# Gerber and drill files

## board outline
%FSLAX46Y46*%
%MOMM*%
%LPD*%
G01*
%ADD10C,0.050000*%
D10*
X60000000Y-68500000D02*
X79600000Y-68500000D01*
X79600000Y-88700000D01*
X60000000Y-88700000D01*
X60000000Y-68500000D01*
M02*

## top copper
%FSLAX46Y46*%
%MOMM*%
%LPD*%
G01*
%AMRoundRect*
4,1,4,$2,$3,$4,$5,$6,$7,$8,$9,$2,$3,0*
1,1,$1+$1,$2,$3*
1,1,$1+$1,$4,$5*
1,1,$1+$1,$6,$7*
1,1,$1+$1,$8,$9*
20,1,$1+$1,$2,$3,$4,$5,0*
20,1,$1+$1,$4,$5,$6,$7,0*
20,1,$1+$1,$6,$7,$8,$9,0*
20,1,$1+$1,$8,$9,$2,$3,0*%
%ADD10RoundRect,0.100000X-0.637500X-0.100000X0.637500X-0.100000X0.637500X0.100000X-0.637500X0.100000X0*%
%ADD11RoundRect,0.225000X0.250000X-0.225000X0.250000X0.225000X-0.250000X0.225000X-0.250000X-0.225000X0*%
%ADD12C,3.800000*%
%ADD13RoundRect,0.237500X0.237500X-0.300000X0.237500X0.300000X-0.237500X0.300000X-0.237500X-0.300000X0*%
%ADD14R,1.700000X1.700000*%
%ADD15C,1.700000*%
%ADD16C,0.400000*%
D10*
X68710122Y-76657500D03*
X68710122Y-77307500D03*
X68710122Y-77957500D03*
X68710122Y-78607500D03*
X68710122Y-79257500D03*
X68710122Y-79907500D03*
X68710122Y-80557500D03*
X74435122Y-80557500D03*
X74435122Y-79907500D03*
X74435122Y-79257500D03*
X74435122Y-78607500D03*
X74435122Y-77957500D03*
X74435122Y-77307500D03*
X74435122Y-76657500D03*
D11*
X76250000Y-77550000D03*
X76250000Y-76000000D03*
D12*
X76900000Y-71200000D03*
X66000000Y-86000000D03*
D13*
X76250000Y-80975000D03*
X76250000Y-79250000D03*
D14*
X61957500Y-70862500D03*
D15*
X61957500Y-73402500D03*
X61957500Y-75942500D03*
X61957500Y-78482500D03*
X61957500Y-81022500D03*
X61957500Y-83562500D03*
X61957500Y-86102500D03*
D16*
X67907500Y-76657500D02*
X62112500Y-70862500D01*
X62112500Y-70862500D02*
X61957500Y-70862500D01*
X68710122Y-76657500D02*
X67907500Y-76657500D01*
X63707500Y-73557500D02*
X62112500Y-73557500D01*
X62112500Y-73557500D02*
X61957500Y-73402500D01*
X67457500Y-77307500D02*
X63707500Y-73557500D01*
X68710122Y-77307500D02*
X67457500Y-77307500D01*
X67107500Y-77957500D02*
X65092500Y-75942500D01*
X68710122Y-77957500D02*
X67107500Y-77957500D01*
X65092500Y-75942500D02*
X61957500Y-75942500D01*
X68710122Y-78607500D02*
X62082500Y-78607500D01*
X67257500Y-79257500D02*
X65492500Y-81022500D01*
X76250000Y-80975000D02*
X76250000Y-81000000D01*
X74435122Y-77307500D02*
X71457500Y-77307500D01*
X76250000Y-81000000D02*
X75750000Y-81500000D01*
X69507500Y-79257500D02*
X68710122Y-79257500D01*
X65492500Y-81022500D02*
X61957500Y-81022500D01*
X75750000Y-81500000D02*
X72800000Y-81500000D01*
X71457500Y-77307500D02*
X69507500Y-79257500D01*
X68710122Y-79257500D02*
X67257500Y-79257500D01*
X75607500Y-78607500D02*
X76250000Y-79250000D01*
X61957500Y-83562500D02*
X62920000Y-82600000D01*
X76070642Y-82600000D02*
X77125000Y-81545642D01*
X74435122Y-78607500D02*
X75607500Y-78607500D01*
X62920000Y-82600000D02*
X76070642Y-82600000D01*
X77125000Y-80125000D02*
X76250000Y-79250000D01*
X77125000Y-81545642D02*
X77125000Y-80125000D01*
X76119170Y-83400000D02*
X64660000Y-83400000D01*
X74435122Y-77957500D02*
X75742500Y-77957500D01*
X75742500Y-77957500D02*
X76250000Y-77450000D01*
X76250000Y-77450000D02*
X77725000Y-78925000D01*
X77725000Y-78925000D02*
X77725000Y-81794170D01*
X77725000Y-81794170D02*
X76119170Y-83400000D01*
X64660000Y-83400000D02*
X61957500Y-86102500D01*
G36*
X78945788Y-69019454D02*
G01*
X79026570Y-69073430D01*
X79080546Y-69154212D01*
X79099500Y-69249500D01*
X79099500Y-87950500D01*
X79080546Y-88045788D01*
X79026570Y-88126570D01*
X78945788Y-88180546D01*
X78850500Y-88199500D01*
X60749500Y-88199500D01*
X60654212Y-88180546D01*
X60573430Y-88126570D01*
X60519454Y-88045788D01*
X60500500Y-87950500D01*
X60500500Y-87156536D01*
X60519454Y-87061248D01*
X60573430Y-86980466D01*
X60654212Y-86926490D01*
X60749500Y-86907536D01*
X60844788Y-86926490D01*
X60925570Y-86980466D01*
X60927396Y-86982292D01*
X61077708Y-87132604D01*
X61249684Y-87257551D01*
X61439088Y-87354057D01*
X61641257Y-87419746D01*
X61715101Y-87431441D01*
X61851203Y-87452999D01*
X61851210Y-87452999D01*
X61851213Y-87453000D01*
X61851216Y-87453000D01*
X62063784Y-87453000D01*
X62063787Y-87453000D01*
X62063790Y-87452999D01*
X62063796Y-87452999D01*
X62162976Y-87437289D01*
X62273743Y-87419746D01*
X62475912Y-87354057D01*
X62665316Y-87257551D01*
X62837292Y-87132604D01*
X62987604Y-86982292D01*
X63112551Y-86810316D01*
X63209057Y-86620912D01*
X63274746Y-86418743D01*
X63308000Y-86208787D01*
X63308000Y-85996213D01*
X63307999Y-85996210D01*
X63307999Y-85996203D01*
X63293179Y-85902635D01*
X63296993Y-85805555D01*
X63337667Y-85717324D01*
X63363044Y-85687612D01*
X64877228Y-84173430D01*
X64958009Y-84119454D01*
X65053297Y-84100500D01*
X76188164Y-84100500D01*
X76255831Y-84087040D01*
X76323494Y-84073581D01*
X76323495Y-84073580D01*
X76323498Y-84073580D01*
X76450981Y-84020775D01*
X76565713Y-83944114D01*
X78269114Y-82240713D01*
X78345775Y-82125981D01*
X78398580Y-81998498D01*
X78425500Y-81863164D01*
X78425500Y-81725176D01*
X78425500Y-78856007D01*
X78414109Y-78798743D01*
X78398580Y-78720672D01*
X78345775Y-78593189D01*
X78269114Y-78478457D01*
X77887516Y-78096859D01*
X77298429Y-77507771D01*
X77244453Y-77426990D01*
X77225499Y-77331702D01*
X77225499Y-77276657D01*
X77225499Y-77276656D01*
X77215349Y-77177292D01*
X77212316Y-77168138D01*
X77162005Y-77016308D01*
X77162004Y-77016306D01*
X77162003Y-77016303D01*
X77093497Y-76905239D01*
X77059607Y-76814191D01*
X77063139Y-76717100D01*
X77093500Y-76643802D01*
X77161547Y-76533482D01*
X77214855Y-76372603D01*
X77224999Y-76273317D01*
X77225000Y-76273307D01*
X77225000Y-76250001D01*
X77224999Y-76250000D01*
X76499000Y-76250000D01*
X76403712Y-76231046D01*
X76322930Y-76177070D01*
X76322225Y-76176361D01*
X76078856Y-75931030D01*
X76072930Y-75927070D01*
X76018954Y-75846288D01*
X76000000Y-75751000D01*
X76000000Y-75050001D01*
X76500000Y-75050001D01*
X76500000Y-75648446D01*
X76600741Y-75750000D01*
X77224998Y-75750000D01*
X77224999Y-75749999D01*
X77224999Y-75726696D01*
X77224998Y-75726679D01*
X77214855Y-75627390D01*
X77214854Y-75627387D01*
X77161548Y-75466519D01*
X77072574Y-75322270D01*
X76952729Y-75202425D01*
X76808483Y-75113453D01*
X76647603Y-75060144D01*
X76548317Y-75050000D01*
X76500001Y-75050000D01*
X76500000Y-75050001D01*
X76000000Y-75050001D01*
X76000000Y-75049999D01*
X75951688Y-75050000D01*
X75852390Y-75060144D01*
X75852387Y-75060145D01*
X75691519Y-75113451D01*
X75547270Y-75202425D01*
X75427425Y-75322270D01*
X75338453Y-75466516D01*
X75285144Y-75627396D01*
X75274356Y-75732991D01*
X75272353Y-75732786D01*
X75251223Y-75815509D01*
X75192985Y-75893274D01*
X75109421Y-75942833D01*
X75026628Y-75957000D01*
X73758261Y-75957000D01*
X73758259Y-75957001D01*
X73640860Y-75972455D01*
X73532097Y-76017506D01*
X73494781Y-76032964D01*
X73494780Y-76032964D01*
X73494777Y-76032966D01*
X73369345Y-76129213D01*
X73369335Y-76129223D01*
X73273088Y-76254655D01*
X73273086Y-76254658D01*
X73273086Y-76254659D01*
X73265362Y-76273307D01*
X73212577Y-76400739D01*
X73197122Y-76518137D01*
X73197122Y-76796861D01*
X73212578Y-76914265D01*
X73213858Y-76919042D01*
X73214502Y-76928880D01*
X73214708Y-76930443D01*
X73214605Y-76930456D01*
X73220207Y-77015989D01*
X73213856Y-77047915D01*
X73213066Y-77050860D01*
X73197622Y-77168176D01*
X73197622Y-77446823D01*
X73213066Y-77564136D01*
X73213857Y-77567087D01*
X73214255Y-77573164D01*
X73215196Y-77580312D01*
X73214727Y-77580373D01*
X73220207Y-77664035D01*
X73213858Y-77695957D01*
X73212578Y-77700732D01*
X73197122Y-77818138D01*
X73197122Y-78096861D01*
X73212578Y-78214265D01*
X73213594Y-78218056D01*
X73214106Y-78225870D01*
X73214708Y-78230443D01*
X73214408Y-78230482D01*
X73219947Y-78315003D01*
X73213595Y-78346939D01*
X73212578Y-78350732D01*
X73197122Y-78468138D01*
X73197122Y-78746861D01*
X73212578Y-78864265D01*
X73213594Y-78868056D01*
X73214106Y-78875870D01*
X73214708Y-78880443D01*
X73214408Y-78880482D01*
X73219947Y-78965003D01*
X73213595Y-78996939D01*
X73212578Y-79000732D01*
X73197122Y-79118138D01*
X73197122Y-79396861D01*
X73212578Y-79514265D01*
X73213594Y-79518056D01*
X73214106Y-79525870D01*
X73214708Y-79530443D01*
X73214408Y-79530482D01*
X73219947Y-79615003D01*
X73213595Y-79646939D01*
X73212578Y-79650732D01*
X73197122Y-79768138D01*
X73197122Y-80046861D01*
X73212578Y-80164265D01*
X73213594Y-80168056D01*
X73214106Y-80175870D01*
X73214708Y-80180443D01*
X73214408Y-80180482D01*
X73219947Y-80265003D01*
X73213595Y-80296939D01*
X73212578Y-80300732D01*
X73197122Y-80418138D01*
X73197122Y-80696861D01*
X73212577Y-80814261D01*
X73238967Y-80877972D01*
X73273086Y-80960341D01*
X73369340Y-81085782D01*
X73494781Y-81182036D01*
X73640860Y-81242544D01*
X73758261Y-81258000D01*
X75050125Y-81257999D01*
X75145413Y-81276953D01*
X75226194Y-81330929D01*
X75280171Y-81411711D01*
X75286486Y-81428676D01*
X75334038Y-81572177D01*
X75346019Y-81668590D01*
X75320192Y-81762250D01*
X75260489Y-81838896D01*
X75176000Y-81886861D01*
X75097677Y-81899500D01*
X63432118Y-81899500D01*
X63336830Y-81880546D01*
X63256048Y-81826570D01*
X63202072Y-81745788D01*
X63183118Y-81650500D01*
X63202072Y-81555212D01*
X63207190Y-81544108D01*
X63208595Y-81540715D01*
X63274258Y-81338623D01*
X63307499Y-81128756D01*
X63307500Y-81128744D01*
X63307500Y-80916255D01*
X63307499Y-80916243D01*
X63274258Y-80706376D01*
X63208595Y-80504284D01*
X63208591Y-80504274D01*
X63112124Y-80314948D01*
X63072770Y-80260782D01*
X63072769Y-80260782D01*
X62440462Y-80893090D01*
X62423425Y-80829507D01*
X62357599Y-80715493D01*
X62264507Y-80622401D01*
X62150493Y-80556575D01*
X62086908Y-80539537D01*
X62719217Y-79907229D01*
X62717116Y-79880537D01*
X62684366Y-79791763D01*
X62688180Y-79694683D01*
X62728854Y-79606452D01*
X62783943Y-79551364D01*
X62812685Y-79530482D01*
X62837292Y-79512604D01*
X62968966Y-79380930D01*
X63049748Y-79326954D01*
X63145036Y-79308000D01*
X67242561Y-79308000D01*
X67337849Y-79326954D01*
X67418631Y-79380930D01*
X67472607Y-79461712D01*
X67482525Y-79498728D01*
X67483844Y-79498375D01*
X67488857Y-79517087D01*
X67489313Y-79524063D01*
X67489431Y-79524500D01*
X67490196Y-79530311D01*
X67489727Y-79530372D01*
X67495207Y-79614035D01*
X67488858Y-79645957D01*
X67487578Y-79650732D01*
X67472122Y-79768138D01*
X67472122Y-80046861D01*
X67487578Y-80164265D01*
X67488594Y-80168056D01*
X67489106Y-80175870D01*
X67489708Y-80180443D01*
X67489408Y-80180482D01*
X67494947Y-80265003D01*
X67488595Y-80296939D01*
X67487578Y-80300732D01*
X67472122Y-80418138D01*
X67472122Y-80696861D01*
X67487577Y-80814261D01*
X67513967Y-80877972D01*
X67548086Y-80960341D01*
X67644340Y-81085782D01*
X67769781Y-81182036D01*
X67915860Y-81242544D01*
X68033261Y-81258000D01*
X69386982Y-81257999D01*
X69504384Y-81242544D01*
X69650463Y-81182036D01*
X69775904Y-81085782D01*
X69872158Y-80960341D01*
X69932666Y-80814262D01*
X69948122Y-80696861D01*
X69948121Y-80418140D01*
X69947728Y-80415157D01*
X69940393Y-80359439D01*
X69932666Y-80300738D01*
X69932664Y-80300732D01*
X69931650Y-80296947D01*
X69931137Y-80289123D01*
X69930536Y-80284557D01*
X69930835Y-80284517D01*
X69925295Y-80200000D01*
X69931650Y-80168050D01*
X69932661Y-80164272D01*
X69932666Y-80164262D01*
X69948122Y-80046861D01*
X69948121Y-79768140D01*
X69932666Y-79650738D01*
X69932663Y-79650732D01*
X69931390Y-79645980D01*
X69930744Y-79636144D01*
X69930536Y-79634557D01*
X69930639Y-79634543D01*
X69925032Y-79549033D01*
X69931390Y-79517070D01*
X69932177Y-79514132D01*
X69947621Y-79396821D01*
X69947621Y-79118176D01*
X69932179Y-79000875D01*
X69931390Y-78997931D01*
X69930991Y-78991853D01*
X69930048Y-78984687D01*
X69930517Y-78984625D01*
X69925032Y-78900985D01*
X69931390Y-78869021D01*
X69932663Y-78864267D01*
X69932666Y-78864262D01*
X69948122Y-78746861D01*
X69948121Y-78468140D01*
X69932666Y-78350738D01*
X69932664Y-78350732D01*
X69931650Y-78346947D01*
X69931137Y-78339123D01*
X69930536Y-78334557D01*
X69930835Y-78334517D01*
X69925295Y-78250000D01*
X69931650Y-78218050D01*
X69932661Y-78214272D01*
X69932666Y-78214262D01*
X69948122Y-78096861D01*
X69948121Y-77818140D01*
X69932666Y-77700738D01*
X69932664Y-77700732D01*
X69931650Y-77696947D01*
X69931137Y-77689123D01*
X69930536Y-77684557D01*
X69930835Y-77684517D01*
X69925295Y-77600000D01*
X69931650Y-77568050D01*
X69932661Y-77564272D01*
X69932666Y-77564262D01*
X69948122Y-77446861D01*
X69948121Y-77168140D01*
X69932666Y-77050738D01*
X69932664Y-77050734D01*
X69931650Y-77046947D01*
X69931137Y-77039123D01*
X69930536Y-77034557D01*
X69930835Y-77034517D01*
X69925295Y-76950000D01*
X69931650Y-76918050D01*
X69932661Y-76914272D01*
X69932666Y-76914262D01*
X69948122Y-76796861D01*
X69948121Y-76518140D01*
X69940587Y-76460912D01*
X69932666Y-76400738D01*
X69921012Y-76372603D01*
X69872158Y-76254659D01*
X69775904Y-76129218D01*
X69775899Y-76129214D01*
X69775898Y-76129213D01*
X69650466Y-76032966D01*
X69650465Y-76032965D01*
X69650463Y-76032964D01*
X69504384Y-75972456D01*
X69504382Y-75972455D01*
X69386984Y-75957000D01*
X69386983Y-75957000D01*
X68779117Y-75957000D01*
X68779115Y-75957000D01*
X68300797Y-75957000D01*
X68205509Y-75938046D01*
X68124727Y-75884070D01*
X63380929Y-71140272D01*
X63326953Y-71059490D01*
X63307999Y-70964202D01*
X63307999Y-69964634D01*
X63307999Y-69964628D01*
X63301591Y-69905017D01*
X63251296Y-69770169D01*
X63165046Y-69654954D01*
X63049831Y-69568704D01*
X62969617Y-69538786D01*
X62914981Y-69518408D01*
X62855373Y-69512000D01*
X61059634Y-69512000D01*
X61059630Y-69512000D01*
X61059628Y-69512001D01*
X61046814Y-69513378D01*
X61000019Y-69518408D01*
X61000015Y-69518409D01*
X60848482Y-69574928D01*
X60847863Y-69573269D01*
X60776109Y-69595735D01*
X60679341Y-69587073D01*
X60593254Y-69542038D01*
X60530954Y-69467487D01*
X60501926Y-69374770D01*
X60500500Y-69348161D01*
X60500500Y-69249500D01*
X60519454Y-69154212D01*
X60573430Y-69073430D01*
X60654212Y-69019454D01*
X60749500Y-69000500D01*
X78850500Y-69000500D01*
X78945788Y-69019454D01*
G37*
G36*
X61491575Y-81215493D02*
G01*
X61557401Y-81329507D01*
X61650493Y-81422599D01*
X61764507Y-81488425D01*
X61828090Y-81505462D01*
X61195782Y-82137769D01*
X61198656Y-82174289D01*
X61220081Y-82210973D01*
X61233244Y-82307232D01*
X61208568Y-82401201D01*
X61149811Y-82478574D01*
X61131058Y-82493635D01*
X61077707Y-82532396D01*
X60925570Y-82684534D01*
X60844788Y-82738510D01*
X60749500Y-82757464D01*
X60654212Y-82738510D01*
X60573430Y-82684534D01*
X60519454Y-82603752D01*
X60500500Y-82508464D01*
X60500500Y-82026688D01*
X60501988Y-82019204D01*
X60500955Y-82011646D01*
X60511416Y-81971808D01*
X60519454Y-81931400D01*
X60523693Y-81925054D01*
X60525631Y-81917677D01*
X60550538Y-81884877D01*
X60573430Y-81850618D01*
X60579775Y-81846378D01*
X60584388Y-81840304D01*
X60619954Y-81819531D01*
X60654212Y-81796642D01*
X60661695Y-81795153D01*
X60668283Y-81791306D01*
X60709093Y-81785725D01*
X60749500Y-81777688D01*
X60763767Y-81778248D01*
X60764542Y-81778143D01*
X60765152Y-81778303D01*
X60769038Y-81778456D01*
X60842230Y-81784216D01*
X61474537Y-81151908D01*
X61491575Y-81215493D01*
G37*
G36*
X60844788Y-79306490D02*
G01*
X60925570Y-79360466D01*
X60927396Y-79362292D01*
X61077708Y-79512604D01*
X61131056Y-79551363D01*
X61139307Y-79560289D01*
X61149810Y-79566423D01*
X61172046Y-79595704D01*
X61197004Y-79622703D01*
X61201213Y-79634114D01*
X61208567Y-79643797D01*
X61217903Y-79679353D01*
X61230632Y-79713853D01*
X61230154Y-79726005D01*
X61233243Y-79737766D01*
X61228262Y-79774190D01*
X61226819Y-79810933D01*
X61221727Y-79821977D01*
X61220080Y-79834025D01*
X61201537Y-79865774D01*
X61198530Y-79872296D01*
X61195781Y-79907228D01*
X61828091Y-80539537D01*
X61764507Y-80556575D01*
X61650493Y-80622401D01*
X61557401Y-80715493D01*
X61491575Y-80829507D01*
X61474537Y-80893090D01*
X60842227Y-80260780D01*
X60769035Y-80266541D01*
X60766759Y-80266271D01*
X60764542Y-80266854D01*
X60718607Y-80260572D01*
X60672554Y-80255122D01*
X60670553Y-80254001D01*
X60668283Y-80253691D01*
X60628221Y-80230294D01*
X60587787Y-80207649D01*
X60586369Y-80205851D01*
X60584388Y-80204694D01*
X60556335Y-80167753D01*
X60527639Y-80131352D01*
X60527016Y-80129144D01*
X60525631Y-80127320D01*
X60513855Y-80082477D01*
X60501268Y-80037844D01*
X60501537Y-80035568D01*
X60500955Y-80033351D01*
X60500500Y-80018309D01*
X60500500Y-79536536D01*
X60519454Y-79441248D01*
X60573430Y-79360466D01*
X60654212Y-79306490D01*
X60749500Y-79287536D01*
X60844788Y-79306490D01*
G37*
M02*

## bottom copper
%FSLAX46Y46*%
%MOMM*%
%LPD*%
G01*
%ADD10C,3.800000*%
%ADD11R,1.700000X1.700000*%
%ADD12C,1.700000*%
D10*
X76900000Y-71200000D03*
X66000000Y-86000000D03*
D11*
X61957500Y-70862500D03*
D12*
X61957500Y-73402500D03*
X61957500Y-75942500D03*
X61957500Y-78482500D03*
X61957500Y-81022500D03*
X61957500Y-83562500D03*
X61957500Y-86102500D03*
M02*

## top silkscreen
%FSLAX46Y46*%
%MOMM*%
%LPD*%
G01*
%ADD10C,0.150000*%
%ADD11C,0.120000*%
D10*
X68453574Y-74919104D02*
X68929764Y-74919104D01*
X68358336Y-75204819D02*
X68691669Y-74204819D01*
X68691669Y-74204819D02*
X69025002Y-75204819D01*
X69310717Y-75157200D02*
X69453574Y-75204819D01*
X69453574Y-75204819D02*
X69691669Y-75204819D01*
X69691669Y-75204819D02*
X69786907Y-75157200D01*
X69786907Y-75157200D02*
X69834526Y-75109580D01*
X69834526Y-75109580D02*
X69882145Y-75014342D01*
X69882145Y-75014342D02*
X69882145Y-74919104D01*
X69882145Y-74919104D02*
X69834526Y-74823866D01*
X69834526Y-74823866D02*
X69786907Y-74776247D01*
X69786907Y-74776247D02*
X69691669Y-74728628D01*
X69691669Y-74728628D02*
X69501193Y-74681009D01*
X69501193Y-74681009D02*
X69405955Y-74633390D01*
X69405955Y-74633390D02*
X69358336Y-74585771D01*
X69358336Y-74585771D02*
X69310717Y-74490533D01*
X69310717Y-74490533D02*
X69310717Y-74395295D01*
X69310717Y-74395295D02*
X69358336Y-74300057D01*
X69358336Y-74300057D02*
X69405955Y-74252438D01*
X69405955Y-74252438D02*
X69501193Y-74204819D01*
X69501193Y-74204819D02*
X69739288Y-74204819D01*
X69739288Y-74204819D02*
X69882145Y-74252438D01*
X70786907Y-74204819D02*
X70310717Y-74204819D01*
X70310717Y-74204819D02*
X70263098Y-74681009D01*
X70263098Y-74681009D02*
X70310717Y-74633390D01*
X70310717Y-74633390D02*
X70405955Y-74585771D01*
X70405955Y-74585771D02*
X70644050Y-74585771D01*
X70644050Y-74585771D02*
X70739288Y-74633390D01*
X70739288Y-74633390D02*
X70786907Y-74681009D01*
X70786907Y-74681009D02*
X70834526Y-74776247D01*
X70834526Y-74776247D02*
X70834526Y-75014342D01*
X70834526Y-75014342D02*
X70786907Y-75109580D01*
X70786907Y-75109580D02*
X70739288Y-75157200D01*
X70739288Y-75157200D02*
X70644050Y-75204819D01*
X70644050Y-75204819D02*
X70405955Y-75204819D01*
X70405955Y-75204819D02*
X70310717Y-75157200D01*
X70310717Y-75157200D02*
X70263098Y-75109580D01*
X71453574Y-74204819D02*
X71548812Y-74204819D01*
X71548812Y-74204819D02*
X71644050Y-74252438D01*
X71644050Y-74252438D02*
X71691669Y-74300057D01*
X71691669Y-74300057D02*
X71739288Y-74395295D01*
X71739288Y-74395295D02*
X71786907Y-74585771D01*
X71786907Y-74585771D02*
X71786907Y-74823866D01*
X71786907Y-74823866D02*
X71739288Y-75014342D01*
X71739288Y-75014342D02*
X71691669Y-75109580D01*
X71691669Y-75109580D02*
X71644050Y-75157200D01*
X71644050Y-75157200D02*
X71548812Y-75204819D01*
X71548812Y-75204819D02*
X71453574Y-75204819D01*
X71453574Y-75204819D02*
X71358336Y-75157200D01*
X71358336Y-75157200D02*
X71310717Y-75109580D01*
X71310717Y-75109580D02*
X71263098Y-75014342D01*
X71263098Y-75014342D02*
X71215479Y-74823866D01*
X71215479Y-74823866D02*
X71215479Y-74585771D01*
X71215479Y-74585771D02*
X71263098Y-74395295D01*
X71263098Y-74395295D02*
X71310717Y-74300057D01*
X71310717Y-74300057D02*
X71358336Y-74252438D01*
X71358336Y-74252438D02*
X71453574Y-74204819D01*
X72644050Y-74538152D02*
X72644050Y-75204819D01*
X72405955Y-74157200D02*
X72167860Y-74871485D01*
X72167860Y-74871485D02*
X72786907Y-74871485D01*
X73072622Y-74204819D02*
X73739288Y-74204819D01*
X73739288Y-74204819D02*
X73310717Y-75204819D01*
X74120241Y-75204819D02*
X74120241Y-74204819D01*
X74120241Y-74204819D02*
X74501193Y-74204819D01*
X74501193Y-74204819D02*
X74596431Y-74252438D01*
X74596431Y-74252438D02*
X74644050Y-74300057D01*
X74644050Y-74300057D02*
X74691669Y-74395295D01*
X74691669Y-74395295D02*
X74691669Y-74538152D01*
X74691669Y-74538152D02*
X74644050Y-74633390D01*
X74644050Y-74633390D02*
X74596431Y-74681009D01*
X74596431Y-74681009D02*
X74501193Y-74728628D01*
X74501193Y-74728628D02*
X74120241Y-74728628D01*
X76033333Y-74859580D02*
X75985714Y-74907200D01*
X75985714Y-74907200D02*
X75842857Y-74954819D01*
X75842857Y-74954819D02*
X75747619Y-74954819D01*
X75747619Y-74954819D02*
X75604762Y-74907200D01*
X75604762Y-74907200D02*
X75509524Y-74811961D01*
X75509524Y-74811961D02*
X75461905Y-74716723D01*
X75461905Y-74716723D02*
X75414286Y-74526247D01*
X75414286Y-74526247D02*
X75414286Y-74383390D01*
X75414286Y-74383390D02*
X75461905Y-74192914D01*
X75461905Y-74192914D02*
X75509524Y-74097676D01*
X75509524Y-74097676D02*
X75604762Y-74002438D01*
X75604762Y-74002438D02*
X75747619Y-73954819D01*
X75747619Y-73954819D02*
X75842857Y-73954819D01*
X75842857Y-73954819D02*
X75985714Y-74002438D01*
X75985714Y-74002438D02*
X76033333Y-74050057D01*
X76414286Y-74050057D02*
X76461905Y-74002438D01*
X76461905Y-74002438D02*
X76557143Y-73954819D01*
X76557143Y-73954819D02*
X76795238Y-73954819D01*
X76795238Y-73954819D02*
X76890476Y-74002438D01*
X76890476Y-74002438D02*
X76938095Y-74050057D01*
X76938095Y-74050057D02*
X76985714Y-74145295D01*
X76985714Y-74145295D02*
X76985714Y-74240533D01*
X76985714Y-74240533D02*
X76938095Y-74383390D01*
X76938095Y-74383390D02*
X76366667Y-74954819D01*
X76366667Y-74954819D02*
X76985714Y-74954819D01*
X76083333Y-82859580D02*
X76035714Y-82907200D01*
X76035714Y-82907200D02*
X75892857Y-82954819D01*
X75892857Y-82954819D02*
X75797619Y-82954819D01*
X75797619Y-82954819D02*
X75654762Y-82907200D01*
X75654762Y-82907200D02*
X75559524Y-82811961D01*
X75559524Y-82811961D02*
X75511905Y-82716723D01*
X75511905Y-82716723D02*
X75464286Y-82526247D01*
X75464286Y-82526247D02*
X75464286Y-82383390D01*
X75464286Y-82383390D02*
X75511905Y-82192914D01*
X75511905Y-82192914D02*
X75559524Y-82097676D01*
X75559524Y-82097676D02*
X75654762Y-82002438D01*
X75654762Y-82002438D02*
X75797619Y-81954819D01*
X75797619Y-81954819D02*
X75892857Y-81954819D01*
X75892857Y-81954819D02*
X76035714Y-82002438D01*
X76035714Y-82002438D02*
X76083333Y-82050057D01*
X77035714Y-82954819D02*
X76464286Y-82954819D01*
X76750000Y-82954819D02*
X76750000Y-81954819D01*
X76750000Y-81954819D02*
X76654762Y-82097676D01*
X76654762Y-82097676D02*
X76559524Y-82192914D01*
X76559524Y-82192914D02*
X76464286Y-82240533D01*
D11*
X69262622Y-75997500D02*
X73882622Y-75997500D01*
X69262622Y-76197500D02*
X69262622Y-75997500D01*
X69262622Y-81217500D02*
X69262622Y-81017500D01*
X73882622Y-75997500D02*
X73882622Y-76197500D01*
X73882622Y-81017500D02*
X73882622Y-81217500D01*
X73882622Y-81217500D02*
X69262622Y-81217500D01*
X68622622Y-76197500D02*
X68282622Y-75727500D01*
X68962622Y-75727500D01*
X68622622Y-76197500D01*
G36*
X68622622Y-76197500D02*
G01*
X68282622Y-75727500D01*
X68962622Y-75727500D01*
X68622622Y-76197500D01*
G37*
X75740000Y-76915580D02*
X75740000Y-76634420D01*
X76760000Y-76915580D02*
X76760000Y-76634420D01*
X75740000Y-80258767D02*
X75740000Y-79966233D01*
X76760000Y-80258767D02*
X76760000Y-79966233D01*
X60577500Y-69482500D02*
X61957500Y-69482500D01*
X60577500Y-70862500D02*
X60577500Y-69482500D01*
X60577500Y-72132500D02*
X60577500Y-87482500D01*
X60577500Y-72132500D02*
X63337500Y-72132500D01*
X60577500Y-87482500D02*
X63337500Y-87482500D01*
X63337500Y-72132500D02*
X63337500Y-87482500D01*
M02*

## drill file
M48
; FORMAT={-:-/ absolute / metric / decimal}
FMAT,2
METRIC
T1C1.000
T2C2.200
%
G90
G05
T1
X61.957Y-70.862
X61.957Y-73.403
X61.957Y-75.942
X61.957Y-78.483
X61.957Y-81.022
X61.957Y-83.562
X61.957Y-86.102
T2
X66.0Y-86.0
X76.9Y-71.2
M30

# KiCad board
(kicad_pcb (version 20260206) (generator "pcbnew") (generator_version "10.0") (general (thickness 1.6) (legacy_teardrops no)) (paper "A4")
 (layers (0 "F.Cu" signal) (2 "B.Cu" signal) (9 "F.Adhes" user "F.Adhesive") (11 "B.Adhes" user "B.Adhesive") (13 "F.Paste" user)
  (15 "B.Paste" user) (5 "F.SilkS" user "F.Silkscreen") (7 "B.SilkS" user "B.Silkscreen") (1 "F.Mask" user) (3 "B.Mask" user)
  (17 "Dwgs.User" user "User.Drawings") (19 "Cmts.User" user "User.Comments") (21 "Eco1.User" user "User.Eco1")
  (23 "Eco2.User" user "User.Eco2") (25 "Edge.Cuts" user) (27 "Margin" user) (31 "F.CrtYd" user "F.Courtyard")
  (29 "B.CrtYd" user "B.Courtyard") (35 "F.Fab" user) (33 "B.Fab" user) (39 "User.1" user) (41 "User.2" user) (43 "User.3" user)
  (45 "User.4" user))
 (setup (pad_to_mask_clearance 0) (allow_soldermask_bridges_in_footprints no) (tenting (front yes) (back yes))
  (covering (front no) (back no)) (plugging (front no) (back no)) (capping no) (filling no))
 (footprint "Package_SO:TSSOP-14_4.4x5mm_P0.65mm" (layer "F.Cu") (at 71.572622 78.6075)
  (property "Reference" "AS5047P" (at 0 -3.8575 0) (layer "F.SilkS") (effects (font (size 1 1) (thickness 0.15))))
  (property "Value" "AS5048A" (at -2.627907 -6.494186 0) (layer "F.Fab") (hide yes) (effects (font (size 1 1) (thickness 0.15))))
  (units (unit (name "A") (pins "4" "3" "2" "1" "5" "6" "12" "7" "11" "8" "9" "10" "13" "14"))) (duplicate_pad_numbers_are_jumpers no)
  (fp_line (start -2.31 -2.61) (end 2.31 -2.61) (stroke (width 0.12) (type solid)) (layer "F.SilkS"))
  (fp_line (start -2.31 -2.41) (end -2.31 -2.61) (stroke (width 0.12) (type solid)) (layer "F.SilkS"))
  (fp_line (start -2.31 2.61) (end -2.31 2.41) (stroke (width 0.12) (type solid)) (layer "F.SilkS"))
  (fp_line (start 2.31 -2.61) (end 2.31 -2.41) (stroke (width 0.12) (type solid)) (layer "F.SilkS"))
  (fp_line (start 2.31 2.41) (end 2.31 2.61) (stroke (width 0.12) (type solid)) (layer "F.SilkS"))
  (fp_line (start 2.31 2.61) (end -2.31 2.61) (stroke (width 0.12) (type solid)) (layer "F.SilkS"))
  (fp_poly (pts (xy -2.95 -2.41) (xy -3.29 -2.88) (xy -2.61 -2.88)) (stroke (width 0.12) (type solid)) (fill yes) (layer "F.SilkS"))
  (pad "1" smd roundrect (at -2.8625 -1.95) (size 1.475 0.4) (layers "F.Cu" "F.Mask" "F.Paste") (roundrect_rratio 0.25) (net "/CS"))
  (pad "2" smd roundrect (at -2.8625 -1.3) (size 1.475 0.4) (layers "F.Cu" "F.Mask" "F.Paste") (roundrect_rratio 0.25) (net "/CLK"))
  (pad "3" smd roundrect (at -2.8625 -0.65) (size 1.475 0.4) (layers "F.Cu" "F.Mask" "F.Paste") (roundrect_rratio 0.25) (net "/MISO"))
  (pad "4" smd roundrect (at -2.8625 0) (size 1.475 0.4) (layers "F.Cu" "F.Mask" "F.Paste") (roundrect_rratio 0.25) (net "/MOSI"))
  (pad "5" smd roundrect (at -2.8625 0.65) (size 1.475 0.4) (layers "F.Cu" "F.Mask" "F.Paste") (roundrect_rratio 0.25) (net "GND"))
  (pad "6" smd roundrect (at -2.8625 1.3) (size 1.475 0.4) (layers "F.Cu" "F.Mask" "F.Paste") (roundrect_rratio 0.25)
   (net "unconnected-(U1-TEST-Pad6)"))
  (pad "7" smd roundrect (at -2.8625 1.95) (size 1.475 0.4) (layers "F.Cu" "F.Mask" "F.Paste") (roundrect_rratio 0.25)
   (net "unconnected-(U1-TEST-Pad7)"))
  (pad "8" smd roundrect (at 2.8625 1.95) (size 1.475 0.4) (layers "F.Cu" "F.Mask" "F.Paste") (roundrect_rratio 0.25)
   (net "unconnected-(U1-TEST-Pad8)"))
  (pad "9" smd roundrect (at 2.8625 1.3) (size 1.475 0.4) (layers "F.Cu" "F.Mask" "F.Paste") (roundrect_rratio 0.25)
   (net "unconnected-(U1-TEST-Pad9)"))
  (pad "10" smd roundrect (at 2.8625 0.65) (size 1.475 0.4) (layers "F.Cu" "F.Mask" "F.Paste") (roundrect_rratio 0.25)
   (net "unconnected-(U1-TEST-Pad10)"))
  (pad "11" smd roundrect (at 2.8625 0) (size 1.475 0.4) (layers "F.Cu" "F.Mask" "F.Paste") (roundrect_rratio 0.25) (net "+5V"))
  (pad "12" smd roundrect (at 2.8625 -0.65) (size 1.475 0.4) (layers "F.Cu" "F.Mask" "F.Paste") (roundrect_rratio 0.25) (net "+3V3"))
  (pad "13" smd roundrect (at 2.8625 -1.3) (size 1.475 0.4) (layers "F.Cu" "F.Mask" "F.Paste") (roundrect_rratio 0.25) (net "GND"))
  (pad "14" smd roundrect (at 2.8625 -1.95) (size 1.475 0.4) (layers "F.Cu" "F.Mask" "F.Paste") (roundrect_rratio 0.25)
   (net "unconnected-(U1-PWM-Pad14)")))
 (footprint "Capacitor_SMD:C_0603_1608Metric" (layer "F.Cu") (at 76.25 76.775 90)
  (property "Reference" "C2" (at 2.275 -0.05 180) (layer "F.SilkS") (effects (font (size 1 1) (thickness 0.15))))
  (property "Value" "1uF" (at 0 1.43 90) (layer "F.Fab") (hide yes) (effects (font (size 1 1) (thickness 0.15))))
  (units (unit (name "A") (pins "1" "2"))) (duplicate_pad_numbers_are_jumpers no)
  (fp_line (start -0.14058 -0.51) (end 0.14058 -0.51) (stroke (width 0.12) (type solid)) (layer "F.SilkS"))
  (fp_line (start -0.14058 0.51) (end 0.14058 0.51) (stroke (width 0.12) (type solid)) (layer "F.SilkS"))
  (pad "1" smd roundrect (at -0.775 0 90) (size 0.9 0.95) (layers "F.Cu" "F.Mask" "F.Paste") (roundrect_rratio 0.25) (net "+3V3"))
  (pad "2" smd roundrect (at 0.775 0 90) (size 0.9 0.95) (layers "F.Cu" "F.Mask" "F.Paste") (roundrect_rratio 0.25) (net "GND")))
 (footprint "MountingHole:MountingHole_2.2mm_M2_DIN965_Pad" (layer "F.Cu") (at 76.9 71.2)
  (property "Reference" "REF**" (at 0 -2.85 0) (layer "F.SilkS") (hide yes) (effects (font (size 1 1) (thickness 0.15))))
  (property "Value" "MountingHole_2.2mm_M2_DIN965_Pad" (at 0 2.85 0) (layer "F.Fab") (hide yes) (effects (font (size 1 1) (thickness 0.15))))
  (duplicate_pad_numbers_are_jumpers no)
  (pad "1" thru_hole circle (at 0 0) (size 3.8 3.8) (drill 2.2) (layers "*.Cu" "*.Mask") (remove_unused_layers no) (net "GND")
   (zone_connect 2)))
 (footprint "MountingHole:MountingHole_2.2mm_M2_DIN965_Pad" (layer "F.Cu") (at 66 86)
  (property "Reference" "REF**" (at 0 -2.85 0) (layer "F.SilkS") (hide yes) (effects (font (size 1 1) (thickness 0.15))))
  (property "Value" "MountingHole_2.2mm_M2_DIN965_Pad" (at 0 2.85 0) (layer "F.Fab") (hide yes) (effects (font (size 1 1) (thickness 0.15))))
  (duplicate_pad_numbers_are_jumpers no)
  (pad "1" thru_hole circle (at 0 0) (size 3.8 3.8) (drill 2.2) (layers "*.Cu" "*.Mask") (remove_unused_layers no) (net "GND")
   (zone_connect 2)))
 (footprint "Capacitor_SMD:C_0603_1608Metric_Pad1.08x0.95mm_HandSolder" (layer "F.Cu") (at 76.25 80.1125 90)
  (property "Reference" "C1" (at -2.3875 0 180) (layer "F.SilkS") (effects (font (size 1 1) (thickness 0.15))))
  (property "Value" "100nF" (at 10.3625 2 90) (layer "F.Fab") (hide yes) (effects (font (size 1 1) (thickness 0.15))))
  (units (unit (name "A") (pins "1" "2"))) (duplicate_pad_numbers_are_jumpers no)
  (fp_line (start -0.146267 -0.51) (end 0.146267 -0.51) (stroke (width 0.12) (type solid)) (layer "F.SilkS"))
  (fp_line (start -0.146267 0.51) (end 0.146267 0.51) (stroke (width 0.12) (type solid)) (layer "F.SilkS"))
  (pad "1" smd roundrect (at -0.8625 0 90) (size 1.075 0.95) (layers "F.Cu" "F.Mask" "F.Paste") (roundrect_rratio 0.25) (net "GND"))
  (pad "2" smd roundrect (at 0.8625 0 90) (size 1.075 0.95) (layers "F.Cu" "F.Mask" "F.Paste") (roundrect_rratio 0.25) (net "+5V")))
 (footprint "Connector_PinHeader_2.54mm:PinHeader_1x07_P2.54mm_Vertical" (layer "F.Cu") (at 61.9575 70.8625)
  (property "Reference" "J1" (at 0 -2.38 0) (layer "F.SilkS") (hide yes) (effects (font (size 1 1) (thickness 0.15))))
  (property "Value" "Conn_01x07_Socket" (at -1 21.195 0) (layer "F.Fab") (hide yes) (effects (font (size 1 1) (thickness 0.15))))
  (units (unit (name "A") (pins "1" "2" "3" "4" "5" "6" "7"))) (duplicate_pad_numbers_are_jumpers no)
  (fp_line (start -1.38 -1.38) (end 0 -1.38) (stroke (width 0.12) (type solid)) (layer "F.SilkS"))
  (fp_line (start -1.38 0) (end -1.38 -1.38) (stroke (width 0.12) (type solid)) (layer "F.SilkS"))
  (fp_line (start -1.38 1.27) (end -1.38 16.62) (stroke (width 0.12) (type solid)) (layer "F.SilkS"))
  (fp_line (start -1.38 1.27) (end 1.38 1.27) (stroke (width 0.12) (type solid)) (layer "F.SilkS"))
  (fp_line (start -1.38 16.62) (end 1.38 16.62) (stroke (width 0.12) (type solid)) (layer "F.SilkS"))
  (fp_line (start 1.38 1.27) (end 1.38 16.62) (stroke (width 0.12) (type solid)) (layer "F.SilkS"))
  (pad "1" thru_hole rect (at 0 0) (size 1.7 1.7) (drill 1) (layers "*.Cu" "*.Mask") (remove_unused_layers no) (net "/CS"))
  (pad "2" thru_hole circle (at 0 2.54) (size 1.7 1.7) (drill 1) (layers "*.Cu" "*.Mask") (remove_unused_layers no) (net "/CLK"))
  (pad "3" thru_hole circle (at 0 5.08) (size 1.7 1.7) (drill 1) (layers "*.Cu" "*.Mask") (remove_unused_layers no) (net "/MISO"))
  (pad "4" thru_hole circle (at 0 7.62) (size 1.7 1.7) (drill 1) (layers "*.Cu" "*.Mask") (remove_unused_layers no) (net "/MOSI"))
  (pad "5" thru_hole circle (at 0 10.16) (size 1.7 1.7) (drill 1) (layers "*.Cu" "*.Mask") (remove_unused_layers no) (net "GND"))
  (pad "6" thru_hole circle (at 0 12.7) (size 1.7 1.7) (drill 1) (layers "*.Cu" "*.Mask") (remove_unused_layers no) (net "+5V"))
  (pad "7" thru_hole circle (at 0 15.24) (size 1.7 1.7) (drill 1) (layers "*.Cu" "*.Mask") (remove_unused_layers no) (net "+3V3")))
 (gr_rect (start 60 68.5) (end 79.6 88.7) (stroke (width 0.05) (type default)) (fill no) (layer "Edge.Cuts"))
 (segment (start 67.9075 76.6575) (end 62.1125 70.8625) (width 0.4) (layer "F.Cu") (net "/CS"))
 (segment (start 62.1125 70.8625) (end 61.9575 70.8625) (width 0.4) (layer "F.Cu") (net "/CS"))
 (segment (start 68.710122 76.6575) (end 67.9075 76.6575) (width 0.4) (layer "F.Cu") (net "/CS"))
 (segment (start 63.7075 73.5575) (end 62.1125 73.5575) (width 0.4) (layer "F.Cu") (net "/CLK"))
 (segment (start 62.1125 73.5575) (end 61.9575 73.4025) (width 0.4) (layer "F.Cu") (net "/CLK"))
 (segment (start 67.4575 77.3075) (end 63.7075 73.5575) (width 0.4) (layer "F.Cu") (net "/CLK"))
 (segment (start 68.710122 77.3075) (end 67.4575 77.3075) (width 0.4) (layer "F.Cu") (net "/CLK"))
 (segment (start 67.1075 77.9575) (end 65.0925 75.9425) (width 0.4) (layer "F.Cu") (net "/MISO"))
 (segment (start 68.710122 77.9575) (end 67.1075 77.9575) (width 0.4) (layer "F.Cu") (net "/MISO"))
 (segment (start 65.0925 75.9425) (end 61.9575 75.9425) (width 0.4) (layer "F.Cu") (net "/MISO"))
 (segment (start 68.710122 78.6075) (end 62.0825 78.6075) (width 0.4) (layer "F.Cu") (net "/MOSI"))
 (segment (start 67.2575 79.2575) (end 65.4925 81.0225) (width 0.4) (layer "F.Cu") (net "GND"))
 (segment (start 76.25 80.975) (end 76.25 81) (width 0.4) (layer "F.Cu") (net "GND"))
 (segment (start 74.435122 77.3075) (end 71.4575 77.3075) (width 0.4) (layer "F.Cu") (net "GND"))
 (segment (start 76.25 81) (end 75.75 81.5) (width 0.4) (layer "F.Cu") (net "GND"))
 (segment (start 69.5075 79.2575) (end 68.710122 79.2575) (width 0.4) (layer "F.Cu") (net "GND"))
 (segment (start 65.4925 81.0225) (end 61.9575 81.0225) (width 0.4) (layer "F.Cu") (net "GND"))
 (segment (start 75.75 81.5) (end 72.8 81.5) (width 0.4) (layer "F.Cu") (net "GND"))
 (segment (start 71.4575 77.3075) (end 69.5075 79.2575) (width 0.4) (layer "F.Cu") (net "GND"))
 (segment (start 68.710122 79.2575) (end 67.2575 79.2575) (width 0.4) (layer "F.Cu") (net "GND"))
 (segment (start 75.6075 78.6075) (end 76.25 79.25) (width 0.4) (layer "F.Cu") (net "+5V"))
 (segment (start 61.9575 83.5625) (end 62.92 82.6) (width 0.4) (layer "F.Cu") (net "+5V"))
 (segment (start 76.070642 82.6) (end 77.125 81.545642) (width 0.4) (layer "F.Cu") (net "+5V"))
 (segment (start 74.435122 78.6075) (end 75.6075 78.6075) (width 0.4) (layer "F.Cu") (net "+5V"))
 (segment (start 62.92 82.6) (end 76.070642 82.6) (width 0.4) (layer "F.Cu") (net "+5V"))
 (segment (start 77.125 80.125) (end 76.25 79.25) (width 0.4) (layer "F.Cu") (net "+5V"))
 (segment (start 77.125 81.545642) (end 77.125 80.125) (width 0.4) (layer "F.Cu") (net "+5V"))
 (segment (start 76.11917 83.4) (end 64.66 83.4) (width 0.4) (layer "F.Cu") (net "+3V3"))
 (segment (start 74.435122 77.9575) (end 75.7425 77.9575) (width 0.4) (layer "F.Cu") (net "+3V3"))
 (segment (start 75.7425 77.9575) (end 76.25 77.45) (width 0.4) (layer "F.Cu") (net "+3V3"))
 (segment (start 76.25 77.45) (end 77.725 78.925) (width 0.4) (layer "F.Cu") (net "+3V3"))
 (segment (start 77.725 78.925) (end 77.725 81.79417) (width 0.4) (layer "F.Cu") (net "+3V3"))
 (segment (start 77.725 81.79417) (end 76.11917 83.4) (width 0.4) (layer "F.Cu") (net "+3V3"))
 (segment (start 64.66 83.4) (end 61.9575 86.1025) (width 0.4) (layer "F.Cu") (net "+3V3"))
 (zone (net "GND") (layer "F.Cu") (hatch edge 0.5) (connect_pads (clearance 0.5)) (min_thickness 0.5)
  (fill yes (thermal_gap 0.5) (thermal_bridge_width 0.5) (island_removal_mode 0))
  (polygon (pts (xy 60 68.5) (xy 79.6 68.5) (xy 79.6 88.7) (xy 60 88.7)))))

